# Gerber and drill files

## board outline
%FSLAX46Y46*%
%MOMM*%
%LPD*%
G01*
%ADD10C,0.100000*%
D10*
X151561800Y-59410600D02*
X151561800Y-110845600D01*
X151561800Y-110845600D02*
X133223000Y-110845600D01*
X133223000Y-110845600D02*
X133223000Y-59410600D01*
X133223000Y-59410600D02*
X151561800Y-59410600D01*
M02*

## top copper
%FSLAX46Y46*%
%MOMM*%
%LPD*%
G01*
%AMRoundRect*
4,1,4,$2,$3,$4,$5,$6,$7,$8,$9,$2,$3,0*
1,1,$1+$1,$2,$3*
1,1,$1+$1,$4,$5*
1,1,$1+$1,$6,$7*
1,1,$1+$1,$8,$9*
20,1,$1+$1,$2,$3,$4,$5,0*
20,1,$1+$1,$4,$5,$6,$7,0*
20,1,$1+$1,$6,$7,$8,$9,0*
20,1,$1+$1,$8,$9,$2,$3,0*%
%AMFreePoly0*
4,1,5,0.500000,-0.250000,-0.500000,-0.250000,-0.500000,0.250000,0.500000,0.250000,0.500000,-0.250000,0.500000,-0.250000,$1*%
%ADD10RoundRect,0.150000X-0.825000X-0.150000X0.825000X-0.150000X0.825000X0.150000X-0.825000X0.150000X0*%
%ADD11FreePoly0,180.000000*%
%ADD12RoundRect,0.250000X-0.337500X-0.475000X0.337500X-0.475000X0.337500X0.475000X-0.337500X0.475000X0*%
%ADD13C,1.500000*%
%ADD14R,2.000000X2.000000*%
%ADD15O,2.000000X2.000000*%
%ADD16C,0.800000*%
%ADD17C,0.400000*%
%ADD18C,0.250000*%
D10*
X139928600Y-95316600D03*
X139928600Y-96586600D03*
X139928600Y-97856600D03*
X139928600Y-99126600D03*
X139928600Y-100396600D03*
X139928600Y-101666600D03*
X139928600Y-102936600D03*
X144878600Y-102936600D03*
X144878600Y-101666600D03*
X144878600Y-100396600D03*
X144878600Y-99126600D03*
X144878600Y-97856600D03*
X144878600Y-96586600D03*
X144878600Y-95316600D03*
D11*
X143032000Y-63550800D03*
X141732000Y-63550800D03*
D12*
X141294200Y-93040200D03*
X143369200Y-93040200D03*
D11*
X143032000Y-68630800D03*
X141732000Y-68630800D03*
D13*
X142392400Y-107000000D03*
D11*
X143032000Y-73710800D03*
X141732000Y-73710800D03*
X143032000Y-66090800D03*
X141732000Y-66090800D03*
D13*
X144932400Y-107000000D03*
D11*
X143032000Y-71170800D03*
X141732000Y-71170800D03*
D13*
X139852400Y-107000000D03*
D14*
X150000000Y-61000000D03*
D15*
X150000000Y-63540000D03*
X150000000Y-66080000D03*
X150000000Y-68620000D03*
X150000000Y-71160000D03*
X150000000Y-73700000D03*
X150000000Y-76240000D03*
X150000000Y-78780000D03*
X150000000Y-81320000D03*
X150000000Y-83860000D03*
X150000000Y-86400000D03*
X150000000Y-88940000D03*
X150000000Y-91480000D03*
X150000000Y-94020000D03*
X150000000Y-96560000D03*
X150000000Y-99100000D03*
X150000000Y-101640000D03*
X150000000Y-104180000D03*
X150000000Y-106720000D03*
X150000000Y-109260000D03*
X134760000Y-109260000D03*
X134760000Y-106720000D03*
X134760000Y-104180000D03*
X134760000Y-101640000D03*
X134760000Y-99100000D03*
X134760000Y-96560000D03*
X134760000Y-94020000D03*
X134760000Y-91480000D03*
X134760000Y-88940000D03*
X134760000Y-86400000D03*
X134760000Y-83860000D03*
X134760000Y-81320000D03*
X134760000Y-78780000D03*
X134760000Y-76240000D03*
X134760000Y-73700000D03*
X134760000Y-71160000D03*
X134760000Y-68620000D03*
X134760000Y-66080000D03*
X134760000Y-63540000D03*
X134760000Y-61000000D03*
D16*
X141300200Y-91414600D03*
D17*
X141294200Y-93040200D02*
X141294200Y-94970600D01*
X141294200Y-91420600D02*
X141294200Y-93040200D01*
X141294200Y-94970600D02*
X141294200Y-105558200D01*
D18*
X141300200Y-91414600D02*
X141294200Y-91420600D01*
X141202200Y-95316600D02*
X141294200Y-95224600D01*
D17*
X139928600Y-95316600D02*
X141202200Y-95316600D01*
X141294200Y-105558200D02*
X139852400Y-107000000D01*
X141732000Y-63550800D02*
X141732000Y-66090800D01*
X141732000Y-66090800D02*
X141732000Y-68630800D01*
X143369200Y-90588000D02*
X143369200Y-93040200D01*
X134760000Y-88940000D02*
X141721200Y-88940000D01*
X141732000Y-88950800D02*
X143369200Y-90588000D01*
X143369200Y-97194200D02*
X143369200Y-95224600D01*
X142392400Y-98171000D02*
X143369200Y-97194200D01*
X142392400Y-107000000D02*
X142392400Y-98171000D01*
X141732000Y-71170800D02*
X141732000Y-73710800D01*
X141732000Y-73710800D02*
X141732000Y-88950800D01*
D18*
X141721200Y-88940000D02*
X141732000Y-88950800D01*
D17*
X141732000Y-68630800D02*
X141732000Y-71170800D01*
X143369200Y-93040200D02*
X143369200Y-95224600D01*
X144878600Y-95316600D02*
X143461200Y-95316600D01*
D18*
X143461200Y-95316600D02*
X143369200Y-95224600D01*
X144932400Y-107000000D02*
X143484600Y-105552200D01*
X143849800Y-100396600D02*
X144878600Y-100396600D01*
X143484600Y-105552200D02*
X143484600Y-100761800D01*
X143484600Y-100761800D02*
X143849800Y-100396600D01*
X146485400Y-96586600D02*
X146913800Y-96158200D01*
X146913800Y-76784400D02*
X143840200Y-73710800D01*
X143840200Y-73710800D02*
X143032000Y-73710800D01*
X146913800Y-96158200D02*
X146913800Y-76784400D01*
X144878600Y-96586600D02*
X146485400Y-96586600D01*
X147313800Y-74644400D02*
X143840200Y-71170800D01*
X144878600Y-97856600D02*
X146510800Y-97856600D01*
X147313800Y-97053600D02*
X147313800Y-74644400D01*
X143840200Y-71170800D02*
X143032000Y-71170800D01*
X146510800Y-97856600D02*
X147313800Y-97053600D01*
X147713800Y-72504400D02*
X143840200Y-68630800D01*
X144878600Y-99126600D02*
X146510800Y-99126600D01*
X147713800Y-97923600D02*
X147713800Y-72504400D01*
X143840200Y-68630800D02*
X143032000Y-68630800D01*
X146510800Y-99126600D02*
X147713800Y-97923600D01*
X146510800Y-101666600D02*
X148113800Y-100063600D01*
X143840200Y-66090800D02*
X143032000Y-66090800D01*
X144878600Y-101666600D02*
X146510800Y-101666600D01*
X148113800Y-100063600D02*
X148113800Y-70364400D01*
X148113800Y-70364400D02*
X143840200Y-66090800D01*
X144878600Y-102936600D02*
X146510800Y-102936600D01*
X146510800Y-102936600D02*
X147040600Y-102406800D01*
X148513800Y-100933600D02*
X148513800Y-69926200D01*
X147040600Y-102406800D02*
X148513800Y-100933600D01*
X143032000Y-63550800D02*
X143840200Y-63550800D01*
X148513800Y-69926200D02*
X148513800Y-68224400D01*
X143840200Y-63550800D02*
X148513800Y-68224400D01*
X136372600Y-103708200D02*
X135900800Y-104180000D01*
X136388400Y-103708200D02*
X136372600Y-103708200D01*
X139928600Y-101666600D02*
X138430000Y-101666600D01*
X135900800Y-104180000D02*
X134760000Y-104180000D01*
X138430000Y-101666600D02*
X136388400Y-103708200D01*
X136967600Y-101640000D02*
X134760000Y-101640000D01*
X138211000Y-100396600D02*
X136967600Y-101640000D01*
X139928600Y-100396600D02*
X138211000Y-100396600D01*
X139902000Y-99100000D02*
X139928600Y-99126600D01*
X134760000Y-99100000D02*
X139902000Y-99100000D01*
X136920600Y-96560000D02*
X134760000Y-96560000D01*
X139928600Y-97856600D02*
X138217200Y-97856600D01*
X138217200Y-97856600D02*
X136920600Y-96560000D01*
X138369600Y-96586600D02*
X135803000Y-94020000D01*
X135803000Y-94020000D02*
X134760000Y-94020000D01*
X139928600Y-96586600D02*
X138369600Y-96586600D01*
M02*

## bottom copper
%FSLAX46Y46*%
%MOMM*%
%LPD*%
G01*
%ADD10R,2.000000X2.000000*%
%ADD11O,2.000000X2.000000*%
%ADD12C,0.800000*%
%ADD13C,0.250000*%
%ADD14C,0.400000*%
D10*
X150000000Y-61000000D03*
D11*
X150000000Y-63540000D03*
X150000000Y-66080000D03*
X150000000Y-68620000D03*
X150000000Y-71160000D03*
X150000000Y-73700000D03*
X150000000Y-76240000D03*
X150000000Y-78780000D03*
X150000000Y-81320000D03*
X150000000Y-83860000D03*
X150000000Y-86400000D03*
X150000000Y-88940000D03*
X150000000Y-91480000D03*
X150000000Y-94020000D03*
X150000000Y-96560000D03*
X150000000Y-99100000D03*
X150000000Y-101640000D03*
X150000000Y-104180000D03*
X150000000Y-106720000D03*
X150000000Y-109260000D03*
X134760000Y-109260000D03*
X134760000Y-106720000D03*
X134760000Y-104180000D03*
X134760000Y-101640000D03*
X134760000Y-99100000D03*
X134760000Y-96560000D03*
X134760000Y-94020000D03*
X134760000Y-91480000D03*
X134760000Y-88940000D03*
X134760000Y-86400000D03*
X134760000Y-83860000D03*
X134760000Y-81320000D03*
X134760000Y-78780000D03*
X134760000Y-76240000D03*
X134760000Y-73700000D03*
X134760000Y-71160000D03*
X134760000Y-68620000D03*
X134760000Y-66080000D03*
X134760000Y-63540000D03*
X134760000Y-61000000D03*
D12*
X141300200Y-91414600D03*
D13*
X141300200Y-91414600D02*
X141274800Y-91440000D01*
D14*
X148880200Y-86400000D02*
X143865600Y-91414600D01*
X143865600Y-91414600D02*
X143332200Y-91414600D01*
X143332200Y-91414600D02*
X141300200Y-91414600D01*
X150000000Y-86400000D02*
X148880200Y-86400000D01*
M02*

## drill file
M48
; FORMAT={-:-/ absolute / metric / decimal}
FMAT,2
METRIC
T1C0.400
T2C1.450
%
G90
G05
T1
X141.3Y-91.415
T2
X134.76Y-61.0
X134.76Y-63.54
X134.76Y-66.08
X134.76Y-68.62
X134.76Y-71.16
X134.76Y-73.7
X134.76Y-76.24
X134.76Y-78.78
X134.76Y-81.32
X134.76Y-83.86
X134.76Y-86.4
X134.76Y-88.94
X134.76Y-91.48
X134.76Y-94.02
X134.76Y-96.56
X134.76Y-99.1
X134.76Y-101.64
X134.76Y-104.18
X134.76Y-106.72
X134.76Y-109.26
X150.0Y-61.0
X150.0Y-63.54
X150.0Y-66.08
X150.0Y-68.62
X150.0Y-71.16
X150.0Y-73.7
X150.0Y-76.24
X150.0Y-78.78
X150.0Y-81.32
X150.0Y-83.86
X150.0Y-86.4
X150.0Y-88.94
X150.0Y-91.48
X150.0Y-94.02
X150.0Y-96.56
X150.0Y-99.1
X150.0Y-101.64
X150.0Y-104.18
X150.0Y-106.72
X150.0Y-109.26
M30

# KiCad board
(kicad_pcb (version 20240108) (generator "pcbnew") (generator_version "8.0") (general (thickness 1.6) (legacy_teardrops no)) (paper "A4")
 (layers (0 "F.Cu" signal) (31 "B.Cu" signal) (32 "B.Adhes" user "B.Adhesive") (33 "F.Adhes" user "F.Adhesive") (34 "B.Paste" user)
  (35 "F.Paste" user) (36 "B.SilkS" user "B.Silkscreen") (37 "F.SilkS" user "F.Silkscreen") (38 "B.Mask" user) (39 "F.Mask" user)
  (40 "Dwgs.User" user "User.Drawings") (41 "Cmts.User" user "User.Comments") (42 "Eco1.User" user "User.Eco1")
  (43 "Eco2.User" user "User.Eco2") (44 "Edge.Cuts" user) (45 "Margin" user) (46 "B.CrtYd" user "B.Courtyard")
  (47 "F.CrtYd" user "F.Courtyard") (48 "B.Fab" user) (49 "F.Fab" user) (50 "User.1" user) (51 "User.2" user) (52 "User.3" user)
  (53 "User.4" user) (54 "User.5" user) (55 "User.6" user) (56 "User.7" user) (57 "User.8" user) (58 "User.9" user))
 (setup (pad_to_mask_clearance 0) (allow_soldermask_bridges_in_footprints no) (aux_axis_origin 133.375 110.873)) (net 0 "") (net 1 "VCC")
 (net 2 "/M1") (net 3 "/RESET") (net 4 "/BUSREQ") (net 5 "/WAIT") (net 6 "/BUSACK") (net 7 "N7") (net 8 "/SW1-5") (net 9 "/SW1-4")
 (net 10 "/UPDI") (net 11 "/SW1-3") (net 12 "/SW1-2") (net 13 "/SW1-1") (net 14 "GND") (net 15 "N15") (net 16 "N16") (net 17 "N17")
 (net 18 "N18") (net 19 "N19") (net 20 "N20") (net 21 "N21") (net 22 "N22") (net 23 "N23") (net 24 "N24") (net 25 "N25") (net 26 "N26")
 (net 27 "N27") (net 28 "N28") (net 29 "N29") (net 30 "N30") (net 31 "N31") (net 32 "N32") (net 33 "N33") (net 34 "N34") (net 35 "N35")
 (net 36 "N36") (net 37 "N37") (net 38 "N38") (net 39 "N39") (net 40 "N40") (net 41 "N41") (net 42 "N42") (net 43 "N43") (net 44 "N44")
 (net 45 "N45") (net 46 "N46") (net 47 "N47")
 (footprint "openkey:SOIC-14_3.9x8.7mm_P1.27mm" (layer "F.Cu") (at 142.4036 99.1266)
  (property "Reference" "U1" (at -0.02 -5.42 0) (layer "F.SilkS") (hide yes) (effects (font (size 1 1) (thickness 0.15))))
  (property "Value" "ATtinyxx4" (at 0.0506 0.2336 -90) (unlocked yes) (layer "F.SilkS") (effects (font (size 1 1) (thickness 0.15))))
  (pad "1" smd roundrect (at -2.475 -3.81) (size 1.95 0.6) (layers "F.Cu" "F.Paste" "F.Mask") (roundrect_rratio 0.25) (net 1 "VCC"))
  (pad "2" smd roundrect (at -2.475 -2.54) (size 1.95 0.6) (layers "F.Cu" "F.Paste" "F.Mask") (roundrect_rratio 0.25) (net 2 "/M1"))
  (pad "3" smd roundrect (at -2.475 -1.27) (size 1.95 0.6) (layers "F.Cu" "F.Paste" "F.Mask") (roundrect_rratio 0.25) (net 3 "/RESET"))
  (pad "4" smd roundrect (at -2.475 0) (size 1.95 0.6) (layers "F.Cu" "F.Paste" "F.Mask") (roundrect_rratio 0.25) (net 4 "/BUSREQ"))
  (pad "5" smd roundrect (at -2.475 1.27) (size 1.95 0.6) (layers "F.Cu" "F.Paste" "F.Mask") (roundrect_rratio 0.25) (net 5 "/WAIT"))
  (pad "6" smd roundrect (at -2.475 2.54) (size 1.95 0.6) (layers "F.Cu" "F.Paste" "F.Mask") (roundrect_rratio 0.25) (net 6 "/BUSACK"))
  (pad "7" smd roundrect (at -2.475 3.81) (size 1.95 0.6) (layers "F.Cu" "F.Paste" "F.Mask") (roundrect_rratio 0.25) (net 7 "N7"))
  (pad "8" smd roundrect (at 2.475 3.81) (size 1.95 0.6) (layers "F.Cu" "F.Paste" "F.Mask") (roundrect_rratio 0.25) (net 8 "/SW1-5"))
  (pad "9" smd roundrect (at 2.475 2.54) (size 1.95 0.6) (layers "F.Cu" "F.Paste" "F.Mask") (roundrect_rratio 0.25) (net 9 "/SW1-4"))
  (pad "10" smd roundrect (at 2.475 1.27) (size 1.95 0.6) (layers "F.Cu" "F.Paste" "F.Mask") (roundrect_rratio 0.25) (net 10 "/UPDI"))
  (pad "11" smd roundrect (at 2.475 0) (size 1.95 0.6) (layers "F.Cu" "F.Paste" "F.Mask") (roundrect_rratio 0.25) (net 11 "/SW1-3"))
  (pad "12" smd roundrect (at 2.475 -1.27) (size 1.95 0.6) (layers "F.Cu" "F.Paste" "F.Mask") (roundrect_rratio 0.25) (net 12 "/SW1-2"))
  (pad "13" smd roundrect (at 2.475 -2.54) (size 1.95 0.6) (layers "F.Cu" "F.Paste" "F.Mask") (roundrect_rratio 0.25) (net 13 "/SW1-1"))
  (pad "14" smd roundrect (at 2.475 -3.81) (size 1.95 0.6) (layers "F.Cu" "F.Paste" "F.Mask") (roundrect_rratio 0.25) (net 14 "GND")))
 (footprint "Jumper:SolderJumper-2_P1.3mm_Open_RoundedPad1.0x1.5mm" (layer "F.Cu") (at 142.382 63.5508 180)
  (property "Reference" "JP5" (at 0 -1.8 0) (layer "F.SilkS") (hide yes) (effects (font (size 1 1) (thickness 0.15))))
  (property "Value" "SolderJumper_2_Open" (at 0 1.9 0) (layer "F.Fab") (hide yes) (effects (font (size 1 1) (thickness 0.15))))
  (pad "1" smd custom (at -0.65 0 180) (size 1 0.5) (layers "F.Cu" "F.Mask") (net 8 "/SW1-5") (zone_connect 2)
   (options (clearance outline) (anchor rect)) (primitives))
  (pad "2" smd custom (at 0.65 0 180) (size 1 0.5) (layers "F.Cu" "F.Mask") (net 14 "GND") (zone_connect 2)
   (options (clearance outline) (anchor rect)) (primitives)))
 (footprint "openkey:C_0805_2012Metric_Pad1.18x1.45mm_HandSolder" (layer "F.Cu") (at 142.3317 93.0402)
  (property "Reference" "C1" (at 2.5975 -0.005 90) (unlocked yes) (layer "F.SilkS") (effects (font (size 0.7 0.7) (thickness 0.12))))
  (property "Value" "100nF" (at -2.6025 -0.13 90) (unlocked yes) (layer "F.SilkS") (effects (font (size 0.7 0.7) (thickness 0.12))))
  (pad "1" smd roundrect (at -1.0375 0) (size 1.175 1.45) (layers "F.Cu" "F.Paste" "F.Mask") (roundrect_rratio 0.212766) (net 1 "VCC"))
  (pad "2" smd roundrect (at 1.0375 0) (size 1.175 1.45) (layers "F.Cu" "F.Paste" "F.Mask") (roundrect_rratio 0.212766) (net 14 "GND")))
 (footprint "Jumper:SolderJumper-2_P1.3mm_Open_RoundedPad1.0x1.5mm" (layer "F.Cu") (at 142.382 68.6308 180)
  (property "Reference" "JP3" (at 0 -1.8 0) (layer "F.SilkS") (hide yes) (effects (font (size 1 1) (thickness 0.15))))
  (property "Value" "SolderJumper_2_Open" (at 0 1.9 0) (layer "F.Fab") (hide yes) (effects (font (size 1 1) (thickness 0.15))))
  (pad "1" smd custom (at -0.65 0 180) (size 1 0.5) (layers "F.Cu" "F.Mask") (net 11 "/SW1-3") (zone_connect 2)
   (options (clearance outline) (anchor rect)) (primitives))
  (pad "2" smd custom (at 0.65 0 180) (size 1 0.5) (layers "F.Cu" "F.Mask") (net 14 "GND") (zone_connect 2)
   (options (clearance outline) (anchor rect)) (primitives)))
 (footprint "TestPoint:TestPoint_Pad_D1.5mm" (layer "F.Cu") (at 142.3924 107 90)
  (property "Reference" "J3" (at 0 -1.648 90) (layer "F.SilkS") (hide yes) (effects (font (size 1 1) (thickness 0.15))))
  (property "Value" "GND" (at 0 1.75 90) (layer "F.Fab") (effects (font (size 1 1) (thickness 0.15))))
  (pad "1" smd circle (at 0 0 90) (size 1.5 1.5) (layers "F.Cu" "F.Mask") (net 14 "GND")))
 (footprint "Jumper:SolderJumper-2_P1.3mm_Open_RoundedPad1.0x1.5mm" (layer "F.Cu") (at 142.382 73.7108 180)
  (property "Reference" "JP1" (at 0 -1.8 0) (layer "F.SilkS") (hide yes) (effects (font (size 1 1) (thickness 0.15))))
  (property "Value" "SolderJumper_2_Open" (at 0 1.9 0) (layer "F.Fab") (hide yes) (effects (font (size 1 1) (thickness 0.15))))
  (pad "1" smd custom (at -0.65 0 180) (size 1 0.5) (layers "F.Cu" "F.Mask") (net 13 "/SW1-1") (zone_connect 2)
   (options (clearance outline) (anchor rect)) (primitives))
  (pad "2" smd custom (at 0.65 0 180) (size 1 0.5) (layers "F.Cu" "F.Mask") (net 14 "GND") (zone_connect 2)
   (options (clearance outline) (anchor rect)) (primitives)))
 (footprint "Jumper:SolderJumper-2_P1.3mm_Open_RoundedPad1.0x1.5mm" (layer "F.Cu") (at 142.382 66.0908 180)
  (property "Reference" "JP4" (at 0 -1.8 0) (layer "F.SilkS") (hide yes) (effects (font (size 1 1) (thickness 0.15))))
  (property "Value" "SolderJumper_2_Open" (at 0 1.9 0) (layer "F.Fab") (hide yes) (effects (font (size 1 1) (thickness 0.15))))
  (pad "1" smd custom (at -0.65 0 180) (size 1 0.5) (layers "F.Cu" "F.Mask") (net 9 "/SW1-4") (zone_connect 2)
   (options (clearance outline) (anchor rect)) (primitives))
  (pad "2" smd custom (at 0.65 0 180) (size 1 0.5) (layers "F.Cu" "F.Mask") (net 14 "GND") (zone_connect 2)
   (options (clearance outline) (anchor rect)) (primitives)))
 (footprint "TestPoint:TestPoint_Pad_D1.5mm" (layer "F.Cu") (at 144.9324 107 90)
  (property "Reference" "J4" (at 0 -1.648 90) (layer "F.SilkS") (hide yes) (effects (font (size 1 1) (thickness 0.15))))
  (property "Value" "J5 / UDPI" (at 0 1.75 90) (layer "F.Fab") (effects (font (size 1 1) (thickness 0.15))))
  (pad "1" smd circle (at 0 0 90) (size 1.5 1.5) (layers "F.Cu" "F.Mask") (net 10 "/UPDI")))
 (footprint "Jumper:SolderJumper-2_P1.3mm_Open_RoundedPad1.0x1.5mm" (layer "F.Cu") (at 142.382 71.1708 180)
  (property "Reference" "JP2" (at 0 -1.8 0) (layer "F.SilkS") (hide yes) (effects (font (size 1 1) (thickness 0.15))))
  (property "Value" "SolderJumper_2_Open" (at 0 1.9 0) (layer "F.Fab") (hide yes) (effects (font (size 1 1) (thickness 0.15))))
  (pad "1" smd custom (at -0.65 0 180) (size 1 0.5) (layers "F.Cu" "F.Mask") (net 12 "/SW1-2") (zone_connect 2)
   (options (clearance outline) (anchor rect)) (primitives))
  (pad "2" smd custom (at 0.65 0 180) (size 1 0.5) (layers "F.Cu" "F.Mask") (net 14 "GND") (zone_connect 2)
   (options (clearance outline) (anchor rect)) (primitives)))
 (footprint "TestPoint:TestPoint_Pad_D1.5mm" (layer "F.Cu") (at 139.8524 107 90)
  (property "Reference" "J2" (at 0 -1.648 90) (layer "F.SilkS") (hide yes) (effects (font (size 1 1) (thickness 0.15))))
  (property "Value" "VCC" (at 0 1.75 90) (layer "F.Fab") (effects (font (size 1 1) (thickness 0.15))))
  (pad "1" smd circle (at 0 0 90) (size 1.5 1.5) (layers "F.Cu" "F.Mask") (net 1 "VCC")))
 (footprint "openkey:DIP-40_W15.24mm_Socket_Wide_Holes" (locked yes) (layer "B.Cu") (at 150 61 180)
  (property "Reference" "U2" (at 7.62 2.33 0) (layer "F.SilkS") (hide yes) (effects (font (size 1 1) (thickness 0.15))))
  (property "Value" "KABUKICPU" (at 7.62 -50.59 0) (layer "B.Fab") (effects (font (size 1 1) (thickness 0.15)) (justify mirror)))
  (pad "1" thru_hole rect (at 0 0 180) (size 2 2) (drill 1.45) (layers "*.Cu" "*.Mask") (remove_unused_layers no) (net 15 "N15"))
  (pad "2" thru_hole oval (at 0 -2.54 180) (size 2 2) (drill 1.45) (layers "*.Cu" "*.Mask") (remove_unused_layers no) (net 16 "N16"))
  (pad "3" thru_hole oval (at 0 -5.08 180) (size 2 2) (drill 1.45) (layers "*.Cu" "*.Mask") (remove_unused_layers no) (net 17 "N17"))
  (pad "4" thru_hole oval (at 0 -7.62 180) (size 2 2) (drill 1.45) (layers "*.Cu" "*.Mask") (remove_unused_layers no) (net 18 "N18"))
  (pad "5" thru_hole oval (at 0 -10.16 180) (size 2 2) (drill 1.45) (layers "*.Cu" "*.Mask") (remove_unused_layers no) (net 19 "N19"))
  (pad "6" thru_hole oval (at 0 -12.7 180) (size 2 2) (drill 1.45) (layers "*.Cu" "*.Mask") (remove_unused_layers no) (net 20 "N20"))
  (pad "7" thru_hole oval (at 0 -15.24 180) (size 2 2) (drill 1.45) (layers "*.Cu" "*.Mask") (remove_unused_layers no) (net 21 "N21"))
  (pad "8" thru_hole oval (at 0 -17.78 180) (size 2 2) (drill 1.45) (layers "*.Cu" "*.Mask") (remove_unused_layers no) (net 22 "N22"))
  (pad "9" thru_hole oval (at 0 -20.32 180) (size 2 2) (drill 1.45) (layers "*.Cu" "*.Mask") (remove_unused_layers no) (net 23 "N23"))
  (pad "10" thru_hole oval (at 0 -22.86 180) (size 2 2) (drill 1.45) (layers "*.Cu" "*.Mask") (remove_unused_layers no) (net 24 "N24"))
  (pad "11" thru_hole oval (at 0 -25.4 180) (size 2 2) (drill 1.45) (layers "*.Cu" "*.Mask") (remove_unused_layers no) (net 1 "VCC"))
  (pad "12" thru_hole oval (at 0 -27.94 180) (size 2 2) (drill 1.45) (layers "*.Cu" "*.Mask") (remove_unused_layers no) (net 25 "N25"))
  (pad "13" thru_hole oval (at 0 -30.48 180) (size 2 2) (drill 1.45) (layers "*.Cu" "*.Mask") (remove_unused_layers no) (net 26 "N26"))
  (pad "14" thru_hole oval (at 0 -33.02 180) (size 2 2) (drill 1.45) (layers "*.Cu" "*.Mask") (remove_unused_layers no) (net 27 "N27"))
  (pad "15" thru_hole oval (at 0 -35.56 180) (size 2 2) (drill 1.45) (layers "*.Cu" "*.Mask") (remove_unused_layers no) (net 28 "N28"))
  (pad "16" thru_hole oval (at 0 -38.1 180) (size 2 2) (drill 1.45) (layers "*.Cu" "*.Mask") (remove_unused_layers no) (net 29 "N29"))
  (pad "17" thru_hole oval (at 0 -40.64 180) (size 2 2) (drill 1.45) (layers "*.Cu" "*.Mask") (remove_unused_layers no) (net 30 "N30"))
  (pad "18" thru_hole oval (at 0 -43.18 180) (size 2 2) (drill 1.45) (layers "*.Cu" "*.Mask") (remove_unused_layers no) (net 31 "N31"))
  (pad "19" thru_hole oval (at 0 -45.72 180) (size 2 2) (drill 1.45) (layers "*.Cu" "*.Mask") (remove_unused_layers no) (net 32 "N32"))
  (pad "20" thru_hole oval (at 0 -48.26 180) (size 2 2) (drill 1.45) (layers "*.Cu" "*.Mask") (remove_unused_layers no) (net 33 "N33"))
  (pad "21" thru_hole oval (at 15.24 -48.26 180) (size 2 2) (drill 1.45) (layers "*.Cu" "*.Mask") (remove_unused_layers no) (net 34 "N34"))
  (pad "22" thru_hole oval (at 15.24 -45.72 180) (size 2 2) (drill 1.45) (layers "*.Cu" "*.Mask") (remove_unused_layers no) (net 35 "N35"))
  (pad "23" thru_hole oval (at 15.24 -43.18 180) (size 2 2) (drill 1.45) (layers "*.Cu" "*.Mask") (remove_unused_layers no)
   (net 6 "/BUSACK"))
  (pad "24" thru_hole oval (at 15.24 -40.64 180) (size 2 2) (drill 1.45) (layers "*.Cu" "*.Mask") (remove_unused_layers no) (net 5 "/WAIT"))
  (pad "25" thru_hole oval (at 15.24 -38.1 180) (size 2 2) (drill 1.45) (layers "*.Cu" "*.Mask") (remove_unused_layers no) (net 4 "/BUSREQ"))
  (pad "26" thru_hole oval (at 15.24 -35.56 180) (size 2 2) (drill 1.45) (layers "*.Cu" "*.Mask") (remove_unused_layers no) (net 3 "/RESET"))
  (pad "27" thru_hole oval (at 15.24 -33.02 180) (size 2 2) (drill 1.45) (layers "*.Cu" "*.Mask") (remove_unused_layers no) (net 2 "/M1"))
  (pad "28" thru_hole oval (at 15.24 -30.48 180) (size 2 2) (drill 1.45) (layers "*.Cu" "*.Mask") (remove_unused_layers no) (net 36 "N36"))
  (pad "29" thru_hole oval (at 15.24 -27.94 180) (size 2 2) (drill 1.45) (layers "*.Cu" "*.Mask") (remove_unused_layers no) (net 14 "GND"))
  (pad "30" thru_hole oval (at 15.24 -25.4 180) (size 2 2) (drill 1.45) (layers "*.Cu" "*.Mask") (remove_unused_layers no) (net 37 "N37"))
  (pad "31" thru_hole oval (at 15.24 -22.86 180) (size 2 2) (drill 1.45) (layers "*.Cu" "*.Mask") (remove_unused_layers no) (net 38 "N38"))
  (pad "32" thru_hole oval (at 15.24 -20.32 180) (size 2 2) (drill 1.45) (layers "*.Cu" "*.Mask") (remove_unused_layers no) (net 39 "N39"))
  (pad "33" thru_hole oval (at 15.24 -17.78 180) (size 2 2) (drill 1.45) (layers "*.Cu" "*.Mask") (remove_unused_layers no) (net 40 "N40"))
  (pad "34" thru_hole oval (at 15.24 -15.24 180) (size 2 2) (drill 1.45) (layers "*.Cu" "*.Mask") (remove_unused_layers no) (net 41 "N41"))
  (pad "35" thru_hole oval (at 15.24 -12.7 180) (size 2 2) (drill 1.45) (layers "*.Cu" "*.Mask") (remove_unused_layers no) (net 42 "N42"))
  (pad "36" thru_hole oval (at 15.24 -10.16 180) (size 2 2) (drill 1.45) (layers "*.Cu" "*.Mask") (remove_unused_layers no) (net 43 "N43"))
  (pad "37" thru_hole oval (at 15.24 -7.62 180) (size 2 2) (drill 1.45) (layers "*.Cu" "*.Mask") (remove_unused_layers no) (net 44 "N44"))
  (pad "38" thru_hole oval (at 15.24 -5.08 180) (size 2 2) (drill 1.45) (layers "*.Cu" "*.Mask") (remove_unused_layers no) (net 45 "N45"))
  (pad "39" thru_hole oval (at 15.24 -2.54 180) (size 2 2) (drill 1.45) (layers "*.Cu" "*.Mask") (remove_unused_layers no) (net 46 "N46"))
  (pad "40" thru_hole oval (at 15.24 0 180) (size 2 2) (drill 1.45) (layers "*.Cu" "*.Mask") (remove_unused_layers no) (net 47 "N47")))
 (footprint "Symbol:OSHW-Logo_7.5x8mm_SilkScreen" (layer "B.Cu") (at 142.375 105.6 180)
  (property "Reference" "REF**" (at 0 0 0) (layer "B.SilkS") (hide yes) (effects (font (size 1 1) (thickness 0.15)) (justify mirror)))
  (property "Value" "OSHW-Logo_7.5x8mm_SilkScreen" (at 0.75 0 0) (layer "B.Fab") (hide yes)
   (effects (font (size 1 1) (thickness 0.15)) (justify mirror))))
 (gr_line (start 151.5618 59.4106) (end 151.5618 110.8456) (stroke (width 0.1) (type solid)) (layer "Edge.Cuts"))
 (gr_line (start 151.5618 110.8456) (end 133.223 110.8456) (stroke (width 0.1) (type solid)) (layer "Edge.Cuts"))
 (gr_line (start 133.223 110.8456) (end 133.223 59.4106) (stroke (width 0.1) (type solid)) (layer "Edge.Cuts"))
 (gr_line (start 133.223 59.4106) (end 151.5618 59.4106) (stroke (width 0.1) (type solid)) (layer "Edge.Cuts"))
 (segment (start 141.2942 93.0402) (end 141.2942 94.9706) (width 0.4) (layer "F.Cu") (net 1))
 (segment (start 141.2942 91.4206) (end 141.2942 93.0402) (width 0.4) (layer "F.Cu") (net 1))
 (segment (start 141.2942 94.9706) (end 141.2942 105.5582) (width 0.4) (layer "F.Cu") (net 1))
 (segment (start 141.3002 91.4146) (end 141.2942 91.4206) (width 0.25) (layer "F.Cu") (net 1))
 (segment (start 141.2022 95.3166) (end 141.2942 95.2246) (width 0.25) (layer "F.Cu") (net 1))
 (segment (start 139.9286 95.3166) (end 141.2022 95.3166) (width 0.4) (layer "F.Cu") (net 1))
 (segment (start 141.2942 105.5582) (end 139.8524 107) (width 0.4) (layer "F.Cu") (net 1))
 (via (at 141.3002 91.4146) (size 0.8) (drill 0.4) (layers "F.Cu" "B.Cu") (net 1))
 (segment (start 141.3002 91.4146) (end 141.2748 91.44) (width 0.25) (layer "B.Cu") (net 1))
 (segment (start 148.8802 86.4) (end 143.8656 91.4146) (width 0.4) (layer "B.Cu") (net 1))
 (segment (start 143.8656 91.4146) (end 143.3322 91.4146) (width 0.4) (layer "B.Cu") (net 1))
 (segment (start 143.3322 91.4146) (end 141.3002 91.4146) (width 0.4) (layer "B.Cu") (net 1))
 (segment (start 150 86.4) (end 148.8802 86.4) (width 0.4) (layer "B.Cu") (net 1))
 (segment (start 141.732 63.5508) (end 141.732 66.0908) (width 0.4) (layer "F.Cu") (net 14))
 (segment (start 141.732 66.0908) (end 141.732 68.6308) (width 0.4) (layer "F.Cu") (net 14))
 (segment (start 143.3692 90.588) (end 143.3692 93.0402) (width 0.4) (layer "F.Cu") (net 14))
 (segment (start 134.76 88.94) (end 141.7212 88.94) (width 0.4) (layer "F.Cu") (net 14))
 (segment (start 141.732 88.9508) (end 143.3692 90.588) (width 0.4) (layer "F.Cu") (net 14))
 (segment (start 143.3692 97.1942) (end 143.3692 95.2246) (width 0.4) (layer "F.Cu") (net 14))
 (segment (start 142.3924 98.171) (end 143.3692 97.1942) (width 0.4) (layer "F.Cu") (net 14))
 (segment (start 142.3924 107) (end 142.3924 98.171) (width 0.4) (layer "F.Cu") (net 14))
 (segment (start 141.732 71.1708) (end 141.732 73.7108) (width 0.4) (layer "F.Cu") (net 14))
 (segment (start 141.732 73.7108) (end 141.732 88.9508) (width 0.4) (layer "F.Cu") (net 14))
 (segment (start 141.7212 88.94) (end 141.732 88.9508) (width 0.25) (layer "F.Cu") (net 14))
 (segment (start 141.732 68.6308) (end 141.732 71.1708) (width 0.4) (layer "F.Cu") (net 14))
 (segment (start 143.3692 93.0402) (end 143.3692 95.2246) (width 0.4) (layer "F.Cu") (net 14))
 (segment (start 144.8786 95.3166) (end 143.4612 95.3166) (width 0.4) (layer "F.Cu") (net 14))
 (segment (start 143.4612 95.3166) (end 143.3692 95.2246) (width 0.25) (layer "F.Cu") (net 14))
 (segment (start 144.9324 107) (end 143.4846 105.5522) (width 0.25) (layer "F.Cu") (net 10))
 (segment (start 143.8498 100.3966) (end 144.8786 100.3966) (width 0.25) (layer "F.Cu") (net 10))
 (segment (start 143.4846 105.5522) (end 143.4846 100.7618) (width 0.25) (layer "F.Cu") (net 10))
 (segment (start 143.4846 100.7618) (end 143.8498 100.3966) (width 0.25) (layer "F.Cu") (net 10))
 (segment (start 146.4854 96.5866) (end 146.9138 96.1582) (width 0.25) (layer "F.Cu") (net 13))
 (segment (start 146.9138 76.7844) (end 143.8402 73.7108) (width 0.25) (layer "F.Cu") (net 13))
 (segment (start 143.8402 73.7108) (end 143.032 73.7108) (width 0.25) (layer "F.Cu") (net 13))
 (segment (start 146.9138 96.1582) (end 146.9138 76.7844) (width 0.25) (layer "F.Cu") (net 13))
 (segment (start 144.8786 96.5866) (end 146.4854 96.5866) (width 0.25) (layer "F.Cu") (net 13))
 (segment (start 147.3138 74.6444) (end 143.8402 71.1708) (width 0.25) (layer "F.Cu") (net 12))
 (segment (start 144.8786 97.8566) (end 146.5108 97.8566) (width 0.25) (layer "F.Cu") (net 12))
 (segment (start 147.3138 97.0536) (end 147.3138 74.6444) (width 0.25) (layer "F.Cu") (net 12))
 (segment (start 143.8402 71.1708) (end 143.032 71.1708) (width 0.25) (layer "F.Cu") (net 12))
 (segment (start 146.5108 97.8566) (end 147.3138 97.0536) (width 0.25) (layer "F.Cu") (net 12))
 (segment (start 147.7138 72.5044) (end 143.8402 68.6308) (width 0.25) (layer "F.Cu") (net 11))
 (segment (start 144.8786 99.1266) (end 146.5108 99.1266) (width 0.25) (layer "F.Cu") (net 11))
 (segment (start 147.7138 97.9236) (end 147.7138 72.5044) (width 0.25) (layer "F.Cu") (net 11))
 (segment (start 143.8402 68.6308) (end 143.032 68.6308) (width 0.25) (layer "F.Cu") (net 11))
 (segment (start 146.5108 99.1266) (end 147.7138 97.9236) (width 0.25) (layer "F.Cu") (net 11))
 (segment (start 146.5108 101.6666) (end 148.1138 100.0636) (width 0.25) (layer "F.Cu") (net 9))
 (segment (start 143.8402 66.0908) (end 143.032 66.0908) (width 0.25) (layer "F.Cu") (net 9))
 (segment (start 144.8786 101.6666) (end 146.5108 101.6666) (width 0.25) (layer "F.Cu") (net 9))
 (segment (start 148.1138 100.0636) (end 148.1138 70.3644) (width 0.25) (layer "F.Cu") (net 9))
 (segment (start 148.1138 70.3644) (end 143.8402 66.0908) (width 0.25) (layer "F.Cu") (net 9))
 (segment (start 144.8786 102.9366) (end 146.5108 102.9366) (width 0.25) (layer "F.Cu") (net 8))
 (segment (start 146.5108 102.9366) (end 147.0406 102.4068) (width 0.25) (layer "F.Cu") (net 8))
 (segment (start 148.5138 100.9336) (end 148.5138 69.9262) (width 0.25) (layer "F.Cu") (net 8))
 (segment (start 147.0406 102.4068) (end 148.5138 100.9336) (width 0.25) (layer "F.Cu") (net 8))
 (segment (start 143.032 63.5508) (end 143.8402 63.5508) (width 0.25) (layer "F.Cu") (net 8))
 (segment (start 148.5138 69.9262) (end 148.5138 68.2244) (width 0.25) (layer "F.Cu") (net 8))
 (segment (start 143.8402 63.5508) (end 148.5138 68.2244) (width 0.25) (layer "F.Cu") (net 8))
 (segment (start 136.3726 103.7082) (end 135.9008 104.18) (width 0.25) (layer "F.Cu") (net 6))
 (segment (start 136.3884 103.7082) (end 136.3726 103.7082) (width 0.25) (layer "F.Cu") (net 6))
 (segment (start 139.9286 101.6666) (end 138.43 101.6666) (width 0.25) (layer "F.Cu") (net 6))
 (segment (start 135.9008 104.18) (end 134.76 104.18) (width 0.25) (layer "F.Cu") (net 6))
 (segment (start 138.43 101.6666) (end 136.3884 103.7082) (width 0.25) (layer "F.Cu") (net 6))
 (segment (start 136.9676 101.64) (end 134.76 101.64) (width 0.25) (layer "F.Cu") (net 5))
 (segment (start 138.211 100.3966) (end 136.9676 101.64) (width 0.25) (layer "F.Cu") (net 5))
 (segment (start 139.9286 100.3966) (end 138.211 100.3966) (width 0.25) (layer "F.Cu") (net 5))
 (segment (start 139.902 99.1) (end 139.9286 99.1266) (width 0.25) (layer "F.Cu") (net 4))
 (segment (start 134.76 99.1) (end 139.902 99.1) (width 0.25) (layer "F.Cu") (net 4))
 (segment (start 136.9206 96.56) (end 134.76 96.56) (width 0.25) (layer "F.Cu") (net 3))
 (segment (start 139.9286 97.8566) (end 138.2172 97.8566) (width 0.25) (layer "F.Cu") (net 3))
 (segment (start 138.2172 97.8566) (end 136.9206 96.56) (width 0.25) (layer "F.Cu") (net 3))
 (segment (start 138.3696 96.5866) (end 135.803 94.02) (width 0.25) (layer "F.Cu") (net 2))
 (segment (start 135.803 94.02) (end 134.76 94.02) (width 0.25) (layer "F.Cu") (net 2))
 (segment (start 139.9286 96.5866) (end 138.3696 96.5866) (width 0.25) (layer "F.Cu") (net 2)))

